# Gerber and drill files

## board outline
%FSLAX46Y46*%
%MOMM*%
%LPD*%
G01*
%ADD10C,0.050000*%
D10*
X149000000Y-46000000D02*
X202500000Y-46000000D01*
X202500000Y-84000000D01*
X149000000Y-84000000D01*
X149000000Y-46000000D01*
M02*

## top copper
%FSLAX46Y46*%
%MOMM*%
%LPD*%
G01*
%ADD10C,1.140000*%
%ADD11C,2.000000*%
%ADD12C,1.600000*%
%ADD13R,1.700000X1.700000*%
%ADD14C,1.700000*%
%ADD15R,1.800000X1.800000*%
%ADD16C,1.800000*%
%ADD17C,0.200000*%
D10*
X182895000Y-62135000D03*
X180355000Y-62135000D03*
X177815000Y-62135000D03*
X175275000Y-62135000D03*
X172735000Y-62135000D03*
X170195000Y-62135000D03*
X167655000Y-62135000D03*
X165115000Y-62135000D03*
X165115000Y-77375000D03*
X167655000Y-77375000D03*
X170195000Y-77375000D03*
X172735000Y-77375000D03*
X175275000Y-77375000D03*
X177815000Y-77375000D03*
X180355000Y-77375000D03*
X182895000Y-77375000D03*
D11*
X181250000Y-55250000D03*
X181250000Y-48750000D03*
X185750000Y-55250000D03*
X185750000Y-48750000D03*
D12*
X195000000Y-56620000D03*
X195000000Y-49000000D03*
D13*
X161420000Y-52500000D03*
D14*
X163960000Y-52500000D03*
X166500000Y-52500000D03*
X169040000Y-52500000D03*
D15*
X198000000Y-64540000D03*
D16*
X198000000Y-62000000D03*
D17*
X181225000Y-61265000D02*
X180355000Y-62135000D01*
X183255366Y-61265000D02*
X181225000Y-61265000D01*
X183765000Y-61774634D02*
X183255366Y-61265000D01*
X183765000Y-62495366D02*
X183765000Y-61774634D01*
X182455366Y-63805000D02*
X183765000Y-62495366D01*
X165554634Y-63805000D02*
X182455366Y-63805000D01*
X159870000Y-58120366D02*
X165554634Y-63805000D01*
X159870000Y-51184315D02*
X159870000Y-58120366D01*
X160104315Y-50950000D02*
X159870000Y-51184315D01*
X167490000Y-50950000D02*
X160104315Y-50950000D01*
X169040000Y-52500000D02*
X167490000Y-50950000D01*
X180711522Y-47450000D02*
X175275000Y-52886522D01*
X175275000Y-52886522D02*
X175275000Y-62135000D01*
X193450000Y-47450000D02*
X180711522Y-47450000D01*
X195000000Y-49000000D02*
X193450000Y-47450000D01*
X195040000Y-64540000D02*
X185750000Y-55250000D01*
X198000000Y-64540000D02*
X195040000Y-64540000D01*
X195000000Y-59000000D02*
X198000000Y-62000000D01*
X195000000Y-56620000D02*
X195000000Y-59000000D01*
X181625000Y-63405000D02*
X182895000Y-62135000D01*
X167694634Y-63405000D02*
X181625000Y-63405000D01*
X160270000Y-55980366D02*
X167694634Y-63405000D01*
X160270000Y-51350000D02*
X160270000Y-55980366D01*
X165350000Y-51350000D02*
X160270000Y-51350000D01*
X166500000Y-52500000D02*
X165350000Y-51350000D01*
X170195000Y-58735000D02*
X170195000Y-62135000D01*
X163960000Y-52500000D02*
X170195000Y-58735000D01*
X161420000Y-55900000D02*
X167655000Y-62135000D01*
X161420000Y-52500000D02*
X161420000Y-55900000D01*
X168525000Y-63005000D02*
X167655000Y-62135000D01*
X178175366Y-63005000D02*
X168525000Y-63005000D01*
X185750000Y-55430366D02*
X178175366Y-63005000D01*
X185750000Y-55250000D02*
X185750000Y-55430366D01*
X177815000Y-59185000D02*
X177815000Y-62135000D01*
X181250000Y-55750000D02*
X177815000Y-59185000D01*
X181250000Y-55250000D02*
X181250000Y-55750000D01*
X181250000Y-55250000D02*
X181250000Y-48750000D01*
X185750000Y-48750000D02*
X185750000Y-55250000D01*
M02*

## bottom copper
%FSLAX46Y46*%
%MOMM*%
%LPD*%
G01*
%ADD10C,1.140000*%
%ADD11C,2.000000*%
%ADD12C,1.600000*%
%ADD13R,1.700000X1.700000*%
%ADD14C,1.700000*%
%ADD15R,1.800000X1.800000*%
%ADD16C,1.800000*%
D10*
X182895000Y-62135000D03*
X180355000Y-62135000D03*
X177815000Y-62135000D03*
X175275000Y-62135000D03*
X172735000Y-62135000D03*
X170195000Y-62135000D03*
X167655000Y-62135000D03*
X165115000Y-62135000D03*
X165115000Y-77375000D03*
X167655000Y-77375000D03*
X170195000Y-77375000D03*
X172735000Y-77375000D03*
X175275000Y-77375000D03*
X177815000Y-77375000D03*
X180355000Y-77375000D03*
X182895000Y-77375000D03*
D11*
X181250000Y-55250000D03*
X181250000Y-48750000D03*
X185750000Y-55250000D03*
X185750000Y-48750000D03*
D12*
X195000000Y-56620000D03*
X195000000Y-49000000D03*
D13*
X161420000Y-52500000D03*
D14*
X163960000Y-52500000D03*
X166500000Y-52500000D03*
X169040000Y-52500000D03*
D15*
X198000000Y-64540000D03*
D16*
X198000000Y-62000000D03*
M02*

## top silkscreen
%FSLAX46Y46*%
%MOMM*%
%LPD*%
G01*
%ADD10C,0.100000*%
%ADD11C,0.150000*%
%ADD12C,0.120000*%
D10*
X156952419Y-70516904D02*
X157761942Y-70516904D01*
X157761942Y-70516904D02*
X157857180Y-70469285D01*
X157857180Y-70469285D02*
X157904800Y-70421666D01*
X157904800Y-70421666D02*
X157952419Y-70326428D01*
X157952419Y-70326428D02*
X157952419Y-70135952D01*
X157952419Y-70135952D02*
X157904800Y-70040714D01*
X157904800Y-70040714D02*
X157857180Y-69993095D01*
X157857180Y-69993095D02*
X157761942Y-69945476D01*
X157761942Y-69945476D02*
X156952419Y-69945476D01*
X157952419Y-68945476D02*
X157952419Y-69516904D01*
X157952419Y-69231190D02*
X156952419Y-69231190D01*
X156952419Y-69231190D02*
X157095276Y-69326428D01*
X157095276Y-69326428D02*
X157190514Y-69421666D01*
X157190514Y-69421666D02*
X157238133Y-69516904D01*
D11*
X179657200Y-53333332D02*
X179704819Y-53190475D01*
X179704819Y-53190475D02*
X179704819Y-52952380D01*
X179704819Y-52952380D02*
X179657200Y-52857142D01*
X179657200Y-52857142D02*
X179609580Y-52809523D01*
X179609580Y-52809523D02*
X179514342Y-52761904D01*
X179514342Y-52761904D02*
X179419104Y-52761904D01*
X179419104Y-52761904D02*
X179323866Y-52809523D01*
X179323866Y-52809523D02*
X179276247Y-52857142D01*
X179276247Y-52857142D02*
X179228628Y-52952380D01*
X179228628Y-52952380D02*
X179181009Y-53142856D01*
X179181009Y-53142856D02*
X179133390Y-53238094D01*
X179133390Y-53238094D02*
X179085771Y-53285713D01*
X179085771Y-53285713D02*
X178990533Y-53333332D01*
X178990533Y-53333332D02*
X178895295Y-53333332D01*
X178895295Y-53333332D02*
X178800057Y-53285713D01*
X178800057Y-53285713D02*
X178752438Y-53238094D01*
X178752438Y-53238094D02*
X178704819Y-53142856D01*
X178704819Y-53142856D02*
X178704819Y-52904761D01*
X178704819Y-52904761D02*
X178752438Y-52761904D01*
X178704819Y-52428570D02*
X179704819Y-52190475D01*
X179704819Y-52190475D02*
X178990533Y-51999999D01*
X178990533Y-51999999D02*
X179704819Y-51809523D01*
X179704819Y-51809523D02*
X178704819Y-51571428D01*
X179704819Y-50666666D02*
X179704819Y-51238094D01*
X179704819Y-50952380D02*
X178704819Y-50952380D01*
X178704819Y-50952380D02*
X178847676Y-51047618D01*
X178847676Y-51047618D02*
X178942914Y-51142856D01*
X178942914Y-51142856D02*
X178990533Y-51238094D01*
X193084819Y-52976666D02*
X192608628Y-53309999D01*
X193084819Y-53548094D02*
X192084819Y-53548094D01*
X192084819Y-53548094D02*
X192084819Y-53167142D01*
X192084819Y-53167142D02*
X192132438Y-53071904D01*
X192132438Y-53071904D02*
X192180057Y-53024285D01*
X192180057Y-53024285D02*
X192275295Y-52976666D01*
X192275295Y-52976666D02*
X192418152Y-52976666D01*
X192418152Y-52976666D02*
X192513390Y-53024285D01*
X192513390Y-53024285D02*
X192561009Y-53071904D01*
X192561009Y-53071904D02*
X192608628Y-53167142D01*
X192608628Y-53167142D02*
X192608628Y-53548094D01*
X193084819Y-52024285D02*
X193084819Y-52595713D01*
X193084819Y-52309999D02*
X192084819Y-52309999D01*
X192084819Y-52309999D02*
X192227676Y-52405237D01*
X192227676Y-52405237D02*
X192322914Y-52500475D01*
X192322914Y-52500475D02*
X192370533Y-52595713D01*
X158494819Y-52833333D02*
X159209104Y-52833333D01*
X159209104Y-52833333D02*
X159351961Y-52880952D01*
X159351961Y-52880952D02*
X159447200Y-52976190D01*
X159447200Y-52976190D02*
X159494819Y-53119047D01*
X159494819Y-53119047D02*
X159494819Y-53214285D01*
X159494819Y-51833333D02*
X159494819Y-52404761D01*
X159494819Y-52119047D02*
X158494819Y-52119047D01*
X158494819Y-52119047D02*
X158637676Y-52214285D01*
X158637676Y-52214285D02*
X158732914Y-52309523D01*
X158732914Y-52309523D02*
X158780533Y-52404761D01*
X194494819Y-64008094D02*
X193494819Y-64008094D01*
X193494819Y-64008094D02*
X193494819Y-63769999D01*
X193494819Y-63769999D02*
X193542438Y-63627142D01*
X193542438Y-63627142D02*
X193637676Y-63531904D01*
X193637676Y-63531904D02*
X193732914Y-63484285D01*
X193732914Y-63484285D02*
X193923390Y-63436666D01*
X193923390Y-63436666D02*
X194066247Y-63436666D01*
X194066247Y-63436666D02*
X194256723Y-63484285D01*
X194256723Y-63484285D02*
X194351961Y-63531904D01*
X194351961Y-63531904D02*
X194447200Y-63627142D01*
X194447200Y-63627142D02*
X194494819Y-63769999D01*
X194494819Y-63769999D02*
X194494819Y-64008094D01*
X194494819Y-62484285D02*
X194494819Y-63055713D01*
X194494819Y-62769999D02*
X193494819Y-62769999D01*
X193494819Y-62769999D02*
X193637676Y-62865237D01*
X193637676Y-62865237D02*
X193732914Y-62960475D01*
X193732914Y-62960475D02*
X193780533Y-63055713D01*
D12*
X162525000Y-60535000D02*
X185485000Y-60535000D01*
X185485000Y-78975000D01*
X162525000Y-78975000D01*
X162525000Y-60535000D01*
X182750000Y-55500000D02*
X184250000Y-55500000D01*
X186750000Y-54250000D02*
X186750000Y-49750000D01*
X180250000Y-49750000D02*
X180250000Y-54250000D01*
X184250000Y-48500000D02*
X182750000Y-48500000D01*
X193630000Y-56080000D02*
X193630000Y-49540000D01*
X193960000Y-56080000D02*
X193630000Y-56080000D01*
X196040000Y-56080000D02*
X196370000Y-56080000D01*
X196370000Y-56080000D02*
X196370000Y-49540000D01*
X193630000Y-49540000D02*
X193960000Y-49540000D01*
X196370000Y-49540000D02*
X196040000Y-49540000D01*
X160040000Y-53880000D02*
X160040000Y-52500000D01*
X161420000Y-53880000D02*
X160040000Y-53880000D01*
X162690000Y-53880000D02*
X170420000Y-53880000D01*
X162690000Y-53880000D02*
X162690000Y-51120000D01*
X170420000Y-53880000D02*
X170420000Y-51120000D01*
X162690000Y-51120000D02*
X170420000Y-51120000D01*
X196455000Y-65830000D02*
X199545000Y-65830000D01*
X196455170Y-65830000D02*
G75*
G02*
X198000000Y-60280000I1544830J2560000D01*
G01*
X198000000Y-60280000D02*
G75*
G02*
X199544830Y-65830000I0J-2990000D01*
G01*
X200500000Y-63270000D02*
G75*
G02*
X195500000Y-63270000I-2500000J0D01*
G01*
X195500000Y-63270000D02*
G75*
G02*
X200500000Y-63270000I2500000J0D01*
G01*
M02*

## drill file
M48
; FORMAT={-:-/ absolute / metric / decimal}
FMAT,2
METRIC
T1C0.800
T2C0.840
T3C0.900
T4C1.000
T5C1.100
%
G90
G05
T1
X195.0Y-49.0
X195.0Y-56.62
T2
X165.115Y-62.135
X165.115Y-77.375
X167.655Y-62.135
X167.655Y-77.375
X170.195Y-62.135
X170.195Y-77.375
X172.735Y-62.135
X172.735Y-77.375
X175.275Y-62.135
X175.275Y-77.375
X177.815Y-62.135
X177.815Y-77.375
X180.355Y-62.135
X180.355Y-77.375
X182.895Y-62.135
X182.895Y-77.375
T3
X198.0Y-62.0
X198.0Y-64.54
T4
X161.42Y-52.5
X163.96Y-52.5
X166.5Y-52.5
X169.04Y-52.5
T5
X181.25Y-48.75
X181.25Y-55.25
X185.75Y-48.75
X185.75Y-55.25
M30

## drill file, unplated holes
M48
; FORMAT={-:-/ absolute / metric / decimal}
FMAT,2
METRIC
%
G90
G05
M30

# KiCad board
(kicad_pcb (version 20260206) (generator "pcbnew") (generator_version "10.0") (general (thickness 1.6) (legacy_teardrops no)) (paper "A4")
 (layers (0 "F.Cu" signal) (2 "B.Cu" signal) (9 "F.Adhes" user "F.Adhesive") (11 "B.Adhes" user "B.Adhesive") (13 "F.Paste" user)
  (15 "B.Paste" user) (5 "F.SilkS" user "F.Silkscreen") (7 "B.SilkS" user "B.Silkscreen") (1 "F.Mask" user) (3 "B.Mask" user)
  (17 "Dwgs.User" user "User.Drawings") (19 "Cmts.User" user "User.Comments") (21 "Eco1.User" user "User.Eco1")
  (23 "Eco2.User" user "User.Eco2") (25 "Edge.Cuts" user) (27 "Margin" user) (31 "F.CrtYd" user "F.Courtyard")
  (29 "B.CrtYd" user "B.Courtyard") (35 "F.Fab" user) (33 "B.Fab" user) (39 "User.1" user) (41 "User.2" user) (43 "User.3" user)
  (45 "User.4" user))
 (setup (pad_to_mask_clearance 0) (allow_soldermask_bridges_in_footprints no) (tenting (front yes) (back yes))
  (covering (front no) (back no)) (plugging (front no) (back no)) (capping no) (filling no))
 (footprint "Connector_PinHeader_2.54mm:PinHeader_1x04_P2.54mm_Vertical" (layer "F.Cu") (at 161.42 52.5 90)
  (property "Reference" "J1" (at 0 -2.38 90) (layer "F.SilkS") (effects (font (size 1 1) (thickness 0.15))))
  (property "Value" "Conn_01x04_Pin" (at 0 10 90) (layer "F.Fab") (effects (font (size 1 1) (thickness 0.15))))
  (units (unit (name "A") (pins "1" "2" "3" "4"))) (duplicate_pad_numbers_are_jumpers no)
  (fp_line (start -1.38 -1.38) (end 0 -1.38) (stroke (width 0.12) (type solid)) (layer "F.SilkS"))
  (fp_line (start -1.38 0) (end -1.38 -1.38) (stroke (width 0.12) (type solid)) (layer "F.SilkS"))
  (fp_line (start 1.38 1.27) (end 1.38 9) (stroke (width 0.12) (type solid)) (layer "F.SilkS"))
  (fp_line (start -1.38 1.27) (end 1.38 1.27) (stroke (width 0.12) (type solid)) (layer "F.SilkS"))
  (fp_line (start -1.38 1.27) (end -1.38 9) (stroke (width 0.12) (type solid)) (layer "F.SilkS"))
  (fp_line (start -1.38 9) (end 1.38 9) (stroke (width 0.12) (type solid)) (layer "F.SilkS"))
  (pad "1" thru_hole rect (at 0 0 90) (size 1.7 1.7) (drill 1) (layers "*.Cu" "*.Mask") (remove_unused_layers no) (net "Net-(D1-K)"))
  (pad "2" thru_hole circle (at 0 2.54 90) (size 1.7 1.7) (drill 1) (layers "*.Cu" "*.Mask") (remove_unused_layers no)
   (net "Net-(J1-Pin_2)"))
  (pad "3" thru_hole circle (at 0 5.08 90) (size 1.7 1.7) (drill 1) (layers "*.Cu" "*.Mask") (remove_unused_layers no)
   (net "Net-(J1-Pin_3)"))
  (pad "4" thru_hole circle (at 0 7.62 90) (size 1.7 1.7) (drill 1) (layers "*.Cu" "*.Mask") (remove_unused_layers no)
   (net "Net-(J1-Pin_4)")))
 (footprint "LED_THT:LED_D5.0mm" (layer "F.Cu") (at 198 64.54 90)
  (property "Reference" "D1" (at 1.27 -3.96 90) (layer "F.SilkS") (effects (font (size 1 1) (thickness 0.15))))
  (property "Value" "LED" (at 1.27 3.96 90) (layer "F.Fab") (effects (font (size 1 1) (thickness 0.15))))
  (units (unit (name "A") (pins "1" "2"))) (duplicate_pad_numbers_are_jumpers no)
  (fp_line (start -1.29 -1.545) (end -1.29 1.545) (stroke (width 0.12) (type solid)) (layer "F.SilkS"))
  (fp_arc (start -1.29 -1.54483) (mid 2.071779 -2.880495) (end 4.26 0) (stroke (width 0.12) (type solid)) (layer "F.SilkS"))
  (fp_arc (start 4.26 0) (mid 2.071779 2.880495) (end -1.29 1.54483) (stroke (width 0.12) (type solid)) (layer "F.SilkS"))
  (fp_circle (center 1.27 0) (end 3.77 0) (stroke (width 0.12) (type solid)) (fill no) (layer "F.SilkS"))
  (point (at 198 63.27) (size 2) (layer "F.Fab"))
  (pad "1" thru_hole rect (at 0 0 90) (size 1.8 1.8) (drill 0.9) (layers "*.Cu" "*.Mask") (remove_unused_layers no) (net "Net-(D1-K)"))
  (pad "2" thru_hole circle (at 2.54 0 90) (size 1.8 1.8) (drill 0.9) (layers "*.Cu" "*.Mask") (remove_unused_layers no) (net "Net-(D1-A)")))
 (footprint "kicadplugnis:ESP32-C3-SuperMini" (layer "F.Cu") (at 174.005 69.755 90)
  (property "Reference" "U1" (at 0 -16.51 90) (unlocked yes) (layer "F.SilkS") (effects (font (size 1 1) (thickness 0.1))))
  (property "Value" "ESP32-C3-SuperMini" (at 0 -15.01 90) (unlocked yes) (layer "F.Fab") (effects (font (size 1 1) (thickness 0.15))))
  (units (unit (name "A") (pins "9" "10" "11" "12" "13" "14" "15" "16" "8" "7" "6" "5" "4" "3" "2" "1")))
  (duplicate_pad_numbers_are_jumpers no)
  (fp_rect (start -9.22 -11.48) (end 9.22 11.48) (stroke (width 0.12) (type solid)) (fill no) (layer "F.SilkS"))
  (pad "1" thru_hole circle (at 7.62 8.89 90) (size 1.14 1.14) (drill 0.84) (layers "*.Cu" "*.Mask") (remove_unused_layers no)
   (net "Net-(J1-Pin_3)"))
  (pad "2" thru_hole circle (at 7.62 6.35 90) (size 1.14 1.14) (drill 0.84) (layers "*.Cu" "*.Mask") (remove_unused_layers no)
   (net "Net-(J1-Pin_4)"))
  (pad "3" thru_hole circle (at 7.62 3.81 90) (size 1.14 1.14) (drill 0.84) (layers "*.Cu" "*.Mask") (remove_unused_layers no)
   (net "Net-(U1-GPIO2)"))
  (pad "4" thru_hole circle (at 7.62 1.27 90) (size 1.14 1.14) (drill 0.84) (layers "*.Cu" "*.Mask") (remove_unused_layers no)
   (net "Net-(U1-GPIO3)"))
  (pad "5" thru_hole circle (at 7.62 -1.27 90) (size 1.14 1.14) (drill 0.84) (layers "*.Cu" "*.Mask") (remove_unused_layers no)
   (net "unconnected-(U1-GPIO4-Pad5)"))
  (pad "6" thru_hole circle (at 7.62 -3.81 90) (size 1.14 1.14) (drill 0.84) (layers "*.Cu" "*.Mask") (remove_unused_layers no)
   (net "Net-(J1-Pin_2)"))
  (pad "7" thru_hole circle (at 7.62 -6.35 90) (size 1.14 1.14) (drill 0.84) (layers "*.Cu" "*.Mask") (remove_unused_layers no)
   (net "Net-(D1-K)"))
  (pad "8" thru_hole circle (at 7.62 -8.89 90) (size 1.14 1.14) (drill 0.84) (layers "*.Cu" "*.Mask") (remove_unused_layers no)
   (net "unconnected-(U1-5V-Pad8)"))
  (pad "9" thru_hole circle (at -7.62 -8.89 90) (size 1.14 1.14) (drill 0.84) (layers "*.Cu" "*.Mask") (remove_unused_layers no)
   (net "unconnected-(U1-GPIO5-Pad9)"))
  (pad "10" thru_hole circle (at -7.62 -6.35 90) (size 1.14 1.14) (drill 0.84) (layers "*.Cu" "*.Mask") (remove_unused_layers no)
   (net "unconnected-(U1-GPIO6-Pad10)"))
  (pad "11" thru_hole circle (at -7.62 -3.81 90) (size 1.14 1.14) (drill 0.84) (layers "*.Cu" "*.Mask") (remove_unused_layers no)
   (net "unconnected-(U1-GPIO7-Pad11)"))
  (pad "12" thru_hole circle (at -7.62 -1.27 90) (size 1.14 1.14) (drill 0.84) (layers "*.Cu" "*.Mask") (remove_unused_layers no)
   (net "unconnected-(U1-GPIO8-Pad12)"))
  (pad "13" thru_hole circle (at -7.62 1.27 90) (size 1.14 1.14) (drill 0.84) (layers "*.Cu" "*.Mask") (remove_unused_layers no)
   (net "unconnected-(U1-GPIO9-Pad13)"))
  (pad "14" thru_hole circle (at -7.62 3.81 90) (size 1.14 1.14) (drill 0.84) (layers "*.Cu" "*.Mask") (remove_unused_layers no)
   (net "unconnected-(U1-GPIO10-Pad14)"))
  (pad "15" thru_hole circle (at -7.62 6.35 90) (size 1.14 1.14) (drill 0.84) (layers "*.Cu" "*.Mask") (remove_unused_layers no)
   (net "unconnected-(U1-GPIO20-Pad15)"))
  (pad "16" thru_hole circle (at -7.62 8.89 90) (size 1.14 1.14) (drill 0.84) (layers "*.Cu" "*.Mask") (remove_unused_layers no)
   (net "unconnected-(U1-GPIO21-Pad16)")))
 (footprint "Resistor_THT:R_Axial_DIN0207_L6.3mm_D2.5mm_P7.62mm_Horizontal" (layer "F.Cu") (at 195 56.62 90)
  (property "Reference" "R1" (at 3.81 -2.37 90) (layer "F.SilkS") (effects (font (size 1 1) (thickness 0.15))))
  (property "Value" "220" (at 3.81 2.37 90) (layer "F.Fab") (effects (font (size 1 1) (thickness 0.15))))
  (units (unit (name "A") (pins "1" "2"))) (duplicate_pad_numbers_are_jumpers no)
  (fp_line (start 7.08 -1.37) (end 7.08 -1.04) (stroke (width 0.12) (type solid)) (layer "F.SilkS"))
  (fp_line (start 0.54 -1.37) (end 7.08 -1.37) (stroke (width 0.12) (type solid)) (layer "F.SilkS"))
  (fp_line (start 0.54 -1.04) (end 0.54 -1.37) (stroke (width 0.12) (type solid)) (layer "F.SilkS"))
  (fp_line (start 0.54 1.04) (end 0.54 1.37) (stroke (width 0.12) (type solid)) (layer "F.SilkS"))
  (fp_line (start 7.08 1.37) (end 7.08 1.04) (stroke (width 0.12) (type solid)) (layer "F.SilkS"))
  (fp_line (start 0.54 1.37) (end 7.08 1.37) (stroke (width 0.12) (type solid)) (layer "F.SilkS"))
  (pad "1" thru_hole circle (at 0 0 90) (size 1.6 1.6) (drill 0.8) (layers "*.Cu" "*.Mask") (remove_unused_layers no) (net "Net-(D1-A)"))
  (pad "2" thru_hole circle (at 7.62 0 90) (size 1.6 1.6) (drill 0.8) (layers "*.Cu" "*.Mask") (remove_unused_layers no)
   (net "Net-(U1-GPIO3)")))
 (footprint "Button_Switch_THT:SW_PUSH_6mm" (layer "F.Cu") (at 181.25 55.25 90)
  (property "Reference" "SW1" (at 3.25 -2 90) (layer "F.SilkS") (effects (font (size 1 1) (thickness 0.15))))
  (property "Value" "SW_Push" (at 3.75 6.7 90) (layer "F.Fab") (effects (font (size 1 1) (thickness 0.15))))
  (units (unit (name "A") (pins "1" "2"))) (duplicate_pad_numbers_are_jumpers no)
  (fp_line (start 5.5 -1) (end 1 -1) (stroke (width 0.12) (type solid)) (layer "F.SilkS"))
  (fp_line (start -0.25 1.5) (end -0.25 3) (stroke (width 0.12) (type solid)) (layer "F.SilkS"))
  (fp_line (start 6.75 3) (end 6.75 1.5) (stroke (width 0.12) (type solid)) (layer "F.SilkS"))
  (fp_line (start 1 5.5) (end 5.5 5.5) (stroke (width 0.12) (type solid)) (layer "F.SilkS"))
  (pad "1" thru_hole circle (at 0 0 180) (size 2 2) (drill 1.1) (layers "*.Cu" "*.Mask") (remove_unused_layers no) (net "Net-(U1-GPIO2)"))
  (pad "1" thru_hole circle (at 6.5 0 180) (size 2 2) (drill 1.1) (layers "*.Cu" "*.Mask") (remove_unused_layers no) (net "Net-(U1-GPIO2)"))
  (pad "2" thru_hole circle (at 0 4.5 180) (size 2 2) (drill 1.1) (layers "*.Cu" "*.Mask") (remove_unused_layers no) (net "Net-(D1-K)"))
  (pad "2" thru_hole circle (at 6.5 4.5 180) (size 2 2) (drill 1.1) (layers "*.Cu" "*.Mask") (remove_unused_layers no) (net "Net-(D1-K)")))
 (gr_rect (start 149 46) (end 202.5 84) (stroke (width 0.05) (type default)) (fill no) (layer "Edge.Cuts"))
 (segment (start 181.625 63.405) (end 182.895 62.135) (width 0.2) (layer "F.Cu") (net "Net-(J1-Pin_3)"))
 (segment (start 165.35 51.35) (end 160.27 51.35) (width 0.2) (layer "F.Cu") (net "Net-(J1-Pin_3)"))
 (segment (start 167.694634 63.405) (end 181.625 63.405) (width 0.2) (layer "F.Cu") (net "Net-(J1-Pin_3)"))
 (segment (start 160.27 51.35) (end 160.27 55.980366) (width 0.2) (layer "F.Cu") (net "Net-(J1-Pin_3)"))
 (segment (start 166.5 52.5) (end 165.35 51.35) (width 0.2) (layer "F.Cu") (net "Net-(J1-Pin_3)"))
 (segment (start 160.27 55.980366) (end 167.694634 63.405) (width 0.2) (layer "F.Cu") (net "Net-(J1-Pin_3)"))
 (segment (start 183.765 62.495366) (end 183.765 61.774634) (width 0.2) (layer "F.Cu") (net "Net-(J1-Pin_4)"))
 (segment (start 160.104315 50.95) (end 159.87 51.184315) (width 0.2) (layer "F.Cu") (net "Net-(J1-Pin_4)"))
 (segment (start 169.04 52.5) (end 167.49 50.95) (width 0.2) (layer "F.Cu") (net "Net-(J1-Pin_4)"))
 (segment (start 183.255366 61.265) (end 181.225 61.265) (width 0.2) (layer "F.Cu") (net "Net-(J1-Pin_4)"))
 (segment (start 165.554634 63.805) (end 182.455366 63.805) (width 0.2) (layer "F.Cu") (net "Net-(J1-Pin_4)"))
 (segment (start 159.87 51.184315) (end 159.87 58.120366) (width 0.2) (layer "F.Cu") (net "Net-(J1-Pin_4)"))
 (segment (start 181.225 61.265) (end 180.355 62.135) (width 0.2) (layer "F.Cu") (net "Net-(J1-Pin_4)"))
 (segment (start 167.49 50.95) (end 160.104315 50.95) (width 0.2) (layer "F.Cu") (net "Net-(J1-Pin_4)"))
 (segment (start 182.455366 63.805) (end 183.765 62.495366) (width 0.2) (layer "F.Cu") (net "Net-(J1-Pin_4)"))
 (segment (start 183.765 61.774634) (end 183.255366 61.265) (width 0.2) (layer "F.Cu") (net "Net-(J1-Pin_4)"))
 (segment (start 159.87 58.120366) (end 165.554634 63.805) (width 0.2) (layer "F.Cu") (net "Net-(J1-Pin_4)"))
 (segment (start 170.195 58.735) (end 170.195 62.135) (width 0.2) (layer "F.Cu") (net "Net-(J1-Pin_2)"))
 (segment (start 163.96 52.5) (end 170.195 58.735) (width 0.2) (layer "F.Cu") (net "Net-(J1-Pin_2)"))
 (segment (start 185.75 55.25) (end 185.75 55.430366) (width 0.2) (layer "F.Cu") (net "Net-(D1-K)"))
 (segment (start 185.75 55.430366) (end 178.175366 63.005) (width 0.2) (layer "F.Cu") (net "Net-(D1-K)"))
 (segment (start 185.75 48.75) (end 185.75 55.25) (width 0.2) (layer "F.Cu") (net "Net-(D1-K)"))
 (segment (start 198 64.54) (end 195.04 64.54) (width 0.2) (layer "F.Cu") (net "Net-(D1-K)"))
 (segment (start 161.42 55.9) (end 167.655 62.135) (width 0.2) (layer "F.Cu") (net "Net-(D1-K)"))
 (segment (start 161.42 52.5) (end 161.42 55.9) (width 0.2) (layer "F.Cu") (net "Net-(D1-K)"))
 (segment (start 168.525 63.005) (end 167.655 62.135) (width 0.2) (layer "F.Cu") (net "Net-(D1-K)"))
 (segment (start 195.04 64.54) (end 185.75 55.25) (width 0.2) (layer "F.Cu") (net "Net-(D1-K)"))
 (segment (start 178.175366 63.005) (end 168.525 63.005) (width 0.2) (layer "F.Cu") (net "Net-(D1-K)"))
 (segment (start 195 56.62) (end 195 59) (width 0.2) (layer "F.Cu") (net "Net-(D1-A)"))
 (segment (start 195 59) (end 198 62) (width 0.2) (layer "F.Cu") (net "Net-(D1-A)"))
 (segment (start 195 49) (end 193.45 47.45) (width 0.2) (layer "F.Cu") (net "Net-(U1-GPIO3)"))
 (segment (start 193.45 47.45) (end 180.711522 47.45) (width 0.2) (layer "F.Cu") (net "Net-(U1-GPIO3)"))
 (segment (start 175.275 52.886522) (end 175.275 62.135) (width 0.2) (layer "F.Cu") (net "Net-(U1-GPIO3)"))
 (segment (start 180.711522 47.45) (end 175.275 52.886522) (width 0.2) (layer "F.Cu") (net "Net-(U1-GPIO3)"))
 (segment (start 181.25 55.25) (end 181.25 55.75) (width 0.2) (layer "F.Cu") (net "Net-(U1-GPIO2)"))
 (segment (start 181.25 55.25) (end 181.25 48.75) (width 0.2) (layer "F.Cu") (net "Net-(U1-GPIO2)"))
 (segment (start 177.815 59.185) (end 177.815 62.135) (width 0.2) (layer "F.Cu") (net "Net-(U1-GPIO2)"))
 (segment (start 181.25 55.75) (end 177.815 59.185) (width 0.2) (layer "F.Cu") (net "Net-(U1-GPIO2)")))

